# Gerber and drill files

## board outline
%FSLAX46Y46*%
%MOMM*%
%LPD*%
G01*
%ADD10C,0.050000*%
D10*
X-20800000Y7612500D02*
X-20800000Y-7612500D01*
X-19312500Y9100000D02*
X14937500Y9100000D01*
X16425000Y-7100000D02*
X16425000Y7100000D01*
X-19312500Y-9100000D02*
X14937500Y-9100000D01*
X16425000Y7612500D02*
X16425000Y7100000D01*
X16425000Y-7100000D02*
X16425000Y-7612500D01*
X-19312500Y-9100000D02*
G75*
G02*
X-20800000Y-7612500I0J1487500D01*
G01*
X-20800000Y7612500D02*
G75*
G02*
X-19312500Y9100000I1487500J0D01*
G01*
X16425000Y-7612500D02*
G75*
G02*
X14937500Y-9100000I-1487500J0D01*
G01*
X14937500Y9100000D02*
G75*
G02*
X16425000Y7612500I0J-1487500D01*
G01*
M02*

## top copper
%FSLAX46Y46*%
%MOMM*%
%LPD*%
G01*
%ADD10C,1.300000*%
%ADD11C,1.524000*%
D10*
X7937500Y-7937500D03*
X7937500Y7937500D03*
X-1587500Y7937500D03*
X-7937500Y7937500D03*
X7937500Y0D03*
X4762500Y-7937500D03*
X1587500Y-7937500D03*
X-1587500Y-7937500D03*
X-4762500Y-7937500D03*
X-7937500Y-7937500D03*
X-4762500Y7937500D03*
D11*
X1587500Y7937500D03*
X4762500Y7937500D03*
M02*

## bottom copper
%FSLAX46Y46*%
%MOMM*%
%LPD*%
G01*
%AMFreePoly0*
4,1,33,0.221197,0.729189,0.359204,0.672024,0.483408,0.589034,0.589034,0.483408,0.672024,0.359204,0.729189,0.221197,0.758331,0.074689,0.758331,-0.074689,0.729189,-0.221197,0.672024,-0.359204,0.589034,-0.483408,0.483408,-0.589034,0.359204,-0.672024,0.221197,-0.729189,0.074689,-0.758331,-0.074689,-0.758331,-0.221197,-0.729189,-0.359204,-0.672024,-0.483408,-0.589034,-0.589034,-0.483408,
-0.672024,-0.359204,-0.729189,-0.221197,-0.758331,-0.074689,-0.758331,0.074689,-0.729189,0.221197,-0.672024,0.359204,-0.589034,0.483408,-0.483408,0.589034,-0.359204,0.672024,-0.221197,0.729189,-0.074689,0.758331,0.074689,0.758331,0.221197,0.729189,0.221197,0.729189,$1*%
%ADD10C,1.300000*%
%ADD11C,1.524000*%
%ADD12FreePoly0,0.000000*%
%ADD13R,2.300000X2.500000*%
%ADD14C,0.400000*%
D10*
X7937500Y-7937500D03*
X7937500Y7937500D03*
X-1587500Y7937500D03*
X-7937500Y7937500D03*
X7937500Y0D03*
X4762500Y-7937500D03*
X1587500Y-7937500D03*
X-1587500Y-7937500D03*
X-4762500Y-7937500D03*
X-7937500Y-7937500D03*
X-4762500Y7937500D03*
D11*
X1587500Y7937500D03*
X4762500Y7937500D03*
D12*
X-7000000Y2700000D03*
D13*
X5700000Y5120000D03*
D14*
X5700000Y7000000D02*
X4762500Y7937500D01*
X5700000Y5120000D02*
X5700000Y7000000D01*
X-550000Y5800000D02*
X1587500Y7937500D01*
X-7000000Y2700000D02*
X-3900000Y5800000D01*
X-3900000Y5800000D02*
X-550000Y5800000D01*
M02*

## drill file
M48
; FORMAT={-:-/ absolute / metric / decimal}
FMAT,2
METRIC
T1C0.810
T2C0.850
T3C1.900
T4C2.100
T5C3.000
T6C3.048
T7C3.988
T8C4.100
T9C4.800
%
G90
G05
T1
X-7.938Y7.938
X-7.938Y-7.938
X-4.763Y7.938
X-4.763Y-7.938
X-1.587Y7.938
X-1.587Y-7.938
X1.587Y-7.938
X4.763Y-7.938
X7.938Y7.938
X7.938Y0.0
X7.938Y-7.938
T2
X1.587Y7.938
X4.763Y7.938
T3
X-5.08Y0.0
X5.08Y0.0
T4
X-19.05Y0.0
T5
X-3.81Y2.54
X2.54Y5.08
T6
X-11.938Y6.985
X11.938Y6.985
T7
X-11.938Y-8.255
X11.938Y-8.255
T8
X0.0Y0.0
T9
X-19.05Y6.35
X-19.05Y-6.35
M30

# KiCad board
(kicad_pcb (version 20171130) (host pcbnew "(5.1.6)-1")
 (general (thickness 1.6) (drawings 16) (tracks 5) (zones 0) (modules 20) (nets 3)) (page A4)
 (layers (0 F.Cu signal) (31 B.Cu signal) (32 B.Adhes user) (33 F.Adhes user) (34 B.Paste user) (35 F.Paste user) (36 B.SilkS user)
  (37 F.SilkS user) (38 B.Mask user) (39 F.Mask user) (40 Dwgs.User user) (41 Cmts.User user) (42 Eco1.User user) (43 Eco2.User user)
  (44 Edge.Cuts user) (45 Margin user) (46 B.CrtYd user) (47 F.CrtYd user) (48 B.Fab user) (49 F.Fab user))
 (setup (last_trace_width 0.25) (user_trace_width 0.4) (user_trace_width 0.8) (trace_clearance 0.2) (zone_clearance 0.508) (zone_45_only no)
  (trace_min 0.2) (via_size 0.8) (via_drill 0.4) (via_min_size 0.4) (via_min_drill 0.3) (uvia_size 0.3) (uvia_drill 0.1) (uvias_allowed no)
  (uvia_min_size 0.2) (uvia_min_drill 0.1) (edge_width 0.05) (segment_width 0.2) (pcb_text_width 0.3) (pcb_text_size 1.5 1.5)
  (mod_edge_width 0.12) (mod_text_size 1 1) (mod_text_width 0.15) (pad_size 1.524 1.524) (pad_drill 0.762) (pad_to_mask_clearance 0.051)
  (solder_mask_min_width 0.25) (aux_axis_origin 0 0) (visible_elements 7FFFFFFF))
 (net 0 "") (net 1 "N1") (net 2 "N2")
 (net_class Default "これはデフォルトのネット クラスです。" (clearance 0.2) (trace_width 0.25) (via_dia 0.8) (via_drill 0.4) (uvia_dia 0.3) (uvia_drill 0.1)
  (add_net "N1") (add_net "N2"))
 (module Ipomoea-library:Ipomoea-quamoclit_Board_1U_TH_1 (layer F.Cu) (at 7.9375 7.9375)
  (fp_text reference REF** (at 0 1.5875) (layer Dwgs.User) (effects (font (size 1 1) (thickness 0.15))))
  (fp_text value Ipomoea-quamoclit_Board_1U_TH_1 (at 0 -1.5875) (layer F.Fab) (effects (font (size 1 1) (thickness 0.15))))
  (pad "" thru_hole circle (at 0 0 180) (size 1.3 1.3) (drill 0.81) (layers *.Cu *.Mask)))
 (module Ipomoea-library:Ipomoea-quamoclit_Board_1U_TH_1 (layer F.Cu) (at 7.9375 -7.9375)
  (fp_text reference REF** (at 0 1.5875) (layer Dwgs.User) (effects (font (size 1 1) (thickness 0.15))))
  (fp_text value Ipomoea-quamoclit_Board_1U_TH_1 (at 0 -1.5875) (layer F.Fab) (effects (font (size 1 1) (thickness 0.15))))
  (pad "" thru_hole circle (at 0 0 180) (size 1.3 1.3) (drill 0.81) (layers *.Cu *.Mask)))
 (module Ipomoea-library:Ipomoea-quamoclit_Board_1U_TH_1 (layer F.Cu) (at -1.5875 -7.9375)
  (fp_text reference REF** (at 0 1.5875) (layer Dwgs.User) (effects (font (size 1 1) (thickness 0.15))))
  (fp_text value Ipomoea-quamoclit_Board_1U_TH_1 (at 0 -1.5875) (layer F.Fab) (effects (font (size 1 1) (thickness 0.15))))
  (pad "" thru_hole circle (at 0 0 180) (size 1.3 1.3) (drill 0.81) (layers *.Cu *.Mask)))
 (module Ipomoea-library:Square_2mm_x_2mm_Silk (layer F.Cu) (at 4.7625 -7.9375)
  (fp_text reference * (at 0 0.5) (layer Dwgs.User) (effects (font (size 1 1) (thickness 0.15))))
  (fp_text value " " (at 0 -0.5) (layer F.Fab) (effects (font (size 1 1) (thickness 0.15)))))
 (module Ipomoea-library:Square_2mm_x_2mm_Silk (layer F.Cu) (at 1.5875 -7.9375)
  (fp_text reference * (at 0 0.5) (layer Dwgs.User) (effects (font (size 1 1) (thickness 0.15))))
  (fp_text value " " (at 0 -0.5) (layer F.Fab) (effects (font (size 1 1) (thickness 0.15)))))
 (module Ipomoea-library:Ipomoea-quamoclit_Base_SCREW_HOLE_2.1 (layer F.Cu) (at -19.05 0 180)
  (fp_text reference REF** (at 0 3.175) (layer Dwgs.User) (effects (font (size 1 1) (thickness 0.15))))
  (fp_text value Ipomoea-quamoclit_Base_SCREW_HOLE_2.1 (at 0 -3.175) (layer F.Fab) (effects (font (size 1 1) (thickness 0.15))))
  (pad "" np_thru_hole circle (at 0 0 180) (size 2.1 2.1) (drill 2.1) (layers *.Cu *.Mask)))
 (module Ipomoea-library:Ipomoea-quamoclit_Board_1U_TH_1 (layer F.Cu) (at -7.9375 -7.9375)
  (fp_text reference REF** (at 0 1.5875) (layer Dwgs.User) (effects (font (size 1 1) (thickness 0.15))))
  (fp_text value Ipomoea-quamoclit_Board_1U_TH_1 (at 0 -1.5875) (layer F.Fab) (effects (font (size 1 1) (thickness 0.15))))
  (pad "" thru_hole circle (at 0 0 180) (size 1.3 1.3) (drill 0.81) (layers *.Cu *.Mask)))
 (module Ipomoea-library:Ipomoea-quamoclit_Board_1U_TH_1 (layer F.Cu) (at 7.9375 0)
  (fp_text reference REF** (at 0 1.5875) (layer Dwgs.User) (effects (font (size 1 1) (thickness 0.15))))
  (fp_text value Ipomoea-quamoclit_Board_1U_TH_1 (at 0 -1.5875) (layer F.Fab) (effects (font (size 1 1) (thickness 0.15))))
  (pad "" thru_hole circle (at 0 0 180) (size 1.3 1.3) (drill 0.81) (layers *.Cu *.Mask)))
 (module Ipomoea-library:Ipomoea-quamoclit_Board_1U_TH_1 (layer F.Cu) (at 4.7625 7.9375)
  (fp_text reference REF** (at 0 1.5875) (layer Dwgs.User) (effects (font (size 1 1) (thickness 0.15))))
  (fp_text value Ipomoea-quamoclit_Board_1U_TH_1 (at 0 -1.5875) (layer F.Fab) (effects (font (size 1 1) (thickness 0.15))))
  (pad "" thru_hole circle (at 0 0 180) (size 1.3 1.3) (drill 0.81) (layers *.Cu *.Mask)))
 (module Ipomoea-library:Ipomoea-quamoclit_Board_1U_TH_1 (layer F.Cu) (at 1.5875 7.9375)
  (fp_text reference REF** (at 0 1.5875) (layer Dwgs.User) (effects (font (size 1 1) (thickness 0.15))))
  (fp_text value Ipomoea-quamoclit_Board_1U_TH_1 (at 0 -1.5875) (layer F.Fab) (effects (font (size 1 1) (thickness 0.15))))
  (pad "" thru_hole circle (at 0 0 180) (size 1.3 1.3) (drill 0.81) (layers *.Cu *.Mask)))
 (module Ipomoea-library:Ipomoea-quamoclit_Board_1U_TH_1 (layer F.Cu) (at -1.5875 7.9375)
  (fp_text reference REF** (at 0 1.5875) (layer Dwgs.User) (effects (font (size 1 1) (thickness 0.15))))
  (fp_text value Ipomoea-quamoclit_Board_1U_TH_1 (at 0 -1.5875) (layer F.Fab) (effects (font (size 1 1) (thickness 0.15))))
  (pad "" thru_hole circle (at 0 0 180) (size 1.3 1.3) (drill 0.81) (layers *.Cu *.Mask)))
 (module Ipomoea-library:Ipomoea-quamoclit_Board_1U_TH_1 (layer F.Cu) (at -4.7625 7.9375)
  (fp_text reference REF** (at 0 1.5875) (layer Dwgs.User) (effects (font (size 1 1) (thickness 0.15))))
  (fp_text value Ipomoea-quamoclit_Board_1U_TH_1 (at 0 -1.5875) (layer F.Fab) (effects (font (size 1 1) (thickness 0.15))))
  (pad "" thru_hole circle (at 0 0 180) (size 1.3 1.3) (drill 0.81) (layers *.Cu *.Mask)))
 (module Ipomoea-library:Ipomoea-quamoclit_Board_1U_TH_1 (layer F.Cu) (at -7.9375 7.9375)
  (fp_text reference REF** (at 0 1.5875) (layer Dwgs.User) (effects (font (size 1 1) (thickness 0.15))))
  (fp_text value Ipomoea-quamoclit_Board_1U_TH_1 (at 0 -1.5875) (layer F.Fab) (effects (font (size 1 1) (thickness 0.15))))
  (pad "" thru_hole circle (at 0 0 180) (size 1.3 1.3) (drill 0.81) (layers *.Cu *.Mask)))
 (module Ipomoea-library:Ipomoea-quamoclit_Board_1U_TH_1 (layer F.Cu) (at -4.7625 -7.9375)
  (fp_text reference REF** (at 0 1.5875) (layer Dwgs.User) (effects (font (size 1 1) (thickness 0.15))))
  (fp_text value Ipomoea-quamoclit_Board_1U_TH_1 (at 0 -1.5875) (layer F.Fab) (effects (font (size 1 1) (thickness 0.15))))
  (pad "" thru_hole circle (at 0 0 180) (size 1.3 1.3) (drill 0.81) (layers *.Cu *.Mask)))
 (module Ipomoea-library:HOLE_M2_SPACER (layer F.Cu) (at -19.05 -6.35)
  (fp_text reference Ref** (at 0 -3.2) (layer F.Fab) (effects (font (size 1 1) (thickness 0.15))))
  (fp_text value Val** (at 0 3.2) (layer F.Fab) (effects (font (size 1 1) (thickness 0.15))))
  (pad "" np_thru_hole circle (at 0 0) (size 4.8 4.8) (drill 4.8) (layers *.Cu *.Mask)))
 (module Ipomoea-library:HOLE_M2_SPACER (layer F.Cu) (at -19.05 6.35)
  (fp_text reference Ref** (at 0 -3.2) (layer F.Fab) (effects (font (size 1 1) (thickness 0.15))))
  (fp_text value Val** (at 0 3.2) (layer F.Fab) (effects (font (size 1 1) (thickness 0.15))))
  (pad "" np_thru_hole circle (at 0 0) (size 4.8 4.8) (drill 4.8) (layers *.Cu *.Mask)))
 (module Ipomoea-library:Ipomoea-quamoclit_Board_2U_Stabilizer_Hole (layer F.Cu) (at 0 0)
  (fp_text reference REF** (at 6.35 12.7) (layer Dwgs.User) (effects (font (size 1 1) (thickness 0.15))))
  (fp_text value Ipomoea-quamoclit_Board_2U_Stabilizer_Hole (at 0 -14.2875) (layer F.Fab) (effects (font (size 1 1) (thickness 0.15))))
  (pad "" np_thru_hole circle (at 11.938 8.255) (size 3.9878 3.9878) (drill 3.9878) (layers *.Cu *.Mask))
  (pad "" np_thru_hole circle (at -11.938 8.255) (size 3.9878 3.9878) (drill 3.9878) (layers *.Cu *.Mask))
  (pad "" np_thru_hole circle (at 11.938 -6.985) (size 3.048 3.048) (drill 3.048) (layers *.Cu *.Mask))
  (pad "" np_thru_hole circle (at -11.938 -6.985) (size 3.048 3.048) (drill 3.048) (layers *.Cu *.Mask)))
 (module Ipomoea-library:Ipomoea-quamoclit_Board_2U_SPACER (layer F.Cu) (at 0 0)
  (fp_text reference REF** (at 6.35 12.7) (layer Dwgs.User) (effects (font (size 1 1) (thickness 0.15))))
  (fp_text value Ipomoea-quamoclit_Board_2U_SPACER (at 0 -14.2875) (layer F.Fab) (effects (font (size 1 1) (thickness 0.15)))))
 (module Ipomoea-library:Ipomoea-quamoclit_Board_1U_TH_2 (layer F.Cu) (at 3.175 -7.9375)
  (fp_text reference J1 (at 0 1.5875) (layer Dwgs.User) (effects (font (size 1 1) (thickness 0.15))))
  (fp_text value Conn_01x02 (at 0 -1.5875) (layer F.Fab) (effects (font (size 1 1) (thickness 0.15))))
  (pad 1 thru_hole circle (at -1.5875 0 180) (size 1.524 1.524) (drill 0.85) (layers *.Cu *.Mask) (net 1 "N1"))
  (pad 2 thru_hole circle (at 1.5875 0 180) (size 1.524 1.524) (drill 0.85) (layers *.Cu *.Mask) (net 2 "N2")))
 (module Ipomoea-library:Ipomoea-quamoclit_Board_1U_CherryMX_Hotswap (layer F.Cu) (at 0 0)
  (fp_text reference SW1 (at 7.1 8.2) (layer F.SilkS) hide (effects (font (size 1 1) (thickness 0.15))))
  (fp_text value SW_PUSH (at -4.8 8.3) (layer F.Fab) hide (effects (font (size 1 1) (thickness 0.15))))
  (pad "" np_thru_hole circle (at 0 0 90) (size 4.1 4.1) (drill 4.1) (layers *.Cu *.Mask))
  (pad "" np_thru_hole circle (at 5.08 0) (size 1.9 1.9) (drill 1.9) (layers *.Cu *.Mask))
  (pad "" np_thru_hole circle (at -5.08 0) (size 1.9 1.9) (drill 1.9) (layers *.Cu *.Mask))
  (pad 1 smd custom (at -7 -2.7) (size 1.524 1.524) (layers B.Cu B.Paste B.Mask) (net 1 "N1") (zone_connect 0)
   (options (clearance outline) (anchor circle)) (primitives))
  (pad "" np_thru_hole circle (at 2.54 -5.08 180) (size 3 3) (drill 3) (layers *.Cu *.Mask))
  (pad 2 smd rect (at 5.7 -5.12 180) (size 2.3 2.5) (layers B.Cu B.Paste B.Mask) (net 2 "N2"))
  (pad "" np_thru_hole circle (at -3.81 -2.54 180) (size 3 3) (drill 3) (layers *.Cu *.Mask)))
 (gr_line (start -20.8 -7.6125) (end -20.8 7.6125) (layer Edge.Cuts) (width 0.05))
 (gr_line (start -19.3125 -9.1) (end 14.9375 -9.1) (layer Edge.Cuts) (width 0.05))
 (gr_line (start 16.425 7.1) (end 16.425 -7.1) (layer Edge.Cuts) (width 0.05))
 (gr_line (start -19.3125 9.1) (end 14.9375 9.1) (layer Edge.Cuts) (width 0.05))
 (gr_line (start 16.425 -7.6125) (end 16.425 -7.1) (layer Edge.Cuts) (width 0.05))
 (gr_line (start 16.425 7.1) (end 16.425 7.6125) (layer Edge.Cuts) (width 0.05))
 (gr_arc (start -19.3125 7.6125) (end -20.8 7.6125) (angle -90) (layer Edge.Cuts) (width 0.05))
 (gr_arc (start -19.3125 -7.6125) (end -19.3125 -9.1) (angle -90) (layer Edge.Cuts) (width 0.05))
 (gr_arc (start 14.9375 7.6125) (end 14.9375 9.1) (angle -90) (layer Edge.Cuts) (width 0.05))
 (gr_arc (start 14.9375 -7.6125) (end 16.425 -7.6125) (angle -90) (layer Edge.Cuts) (width 0.05))
 (segment (start 5.7 -7) (end 4.7625 -7.9375) (width 0.4) (layer B.Cu) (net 2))
 (segment (start 5.7 -5.12) (end 5.7 -7) (width 0.4) (layer B.Cu) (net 2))
 (segment (start -0.55 -5.8) (end 1.5875 -7.9375) (width 0.4) (layer B.Cu) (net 1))
 (segment (start -7 -2.7) (end -3.9 -5.8) (width 0.4) (layer B.Cu) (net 1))
 (segment (start -3.9 -5.8) (end -0.55 -5.8) (width 0.4) (layer B.Cu) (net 1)))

